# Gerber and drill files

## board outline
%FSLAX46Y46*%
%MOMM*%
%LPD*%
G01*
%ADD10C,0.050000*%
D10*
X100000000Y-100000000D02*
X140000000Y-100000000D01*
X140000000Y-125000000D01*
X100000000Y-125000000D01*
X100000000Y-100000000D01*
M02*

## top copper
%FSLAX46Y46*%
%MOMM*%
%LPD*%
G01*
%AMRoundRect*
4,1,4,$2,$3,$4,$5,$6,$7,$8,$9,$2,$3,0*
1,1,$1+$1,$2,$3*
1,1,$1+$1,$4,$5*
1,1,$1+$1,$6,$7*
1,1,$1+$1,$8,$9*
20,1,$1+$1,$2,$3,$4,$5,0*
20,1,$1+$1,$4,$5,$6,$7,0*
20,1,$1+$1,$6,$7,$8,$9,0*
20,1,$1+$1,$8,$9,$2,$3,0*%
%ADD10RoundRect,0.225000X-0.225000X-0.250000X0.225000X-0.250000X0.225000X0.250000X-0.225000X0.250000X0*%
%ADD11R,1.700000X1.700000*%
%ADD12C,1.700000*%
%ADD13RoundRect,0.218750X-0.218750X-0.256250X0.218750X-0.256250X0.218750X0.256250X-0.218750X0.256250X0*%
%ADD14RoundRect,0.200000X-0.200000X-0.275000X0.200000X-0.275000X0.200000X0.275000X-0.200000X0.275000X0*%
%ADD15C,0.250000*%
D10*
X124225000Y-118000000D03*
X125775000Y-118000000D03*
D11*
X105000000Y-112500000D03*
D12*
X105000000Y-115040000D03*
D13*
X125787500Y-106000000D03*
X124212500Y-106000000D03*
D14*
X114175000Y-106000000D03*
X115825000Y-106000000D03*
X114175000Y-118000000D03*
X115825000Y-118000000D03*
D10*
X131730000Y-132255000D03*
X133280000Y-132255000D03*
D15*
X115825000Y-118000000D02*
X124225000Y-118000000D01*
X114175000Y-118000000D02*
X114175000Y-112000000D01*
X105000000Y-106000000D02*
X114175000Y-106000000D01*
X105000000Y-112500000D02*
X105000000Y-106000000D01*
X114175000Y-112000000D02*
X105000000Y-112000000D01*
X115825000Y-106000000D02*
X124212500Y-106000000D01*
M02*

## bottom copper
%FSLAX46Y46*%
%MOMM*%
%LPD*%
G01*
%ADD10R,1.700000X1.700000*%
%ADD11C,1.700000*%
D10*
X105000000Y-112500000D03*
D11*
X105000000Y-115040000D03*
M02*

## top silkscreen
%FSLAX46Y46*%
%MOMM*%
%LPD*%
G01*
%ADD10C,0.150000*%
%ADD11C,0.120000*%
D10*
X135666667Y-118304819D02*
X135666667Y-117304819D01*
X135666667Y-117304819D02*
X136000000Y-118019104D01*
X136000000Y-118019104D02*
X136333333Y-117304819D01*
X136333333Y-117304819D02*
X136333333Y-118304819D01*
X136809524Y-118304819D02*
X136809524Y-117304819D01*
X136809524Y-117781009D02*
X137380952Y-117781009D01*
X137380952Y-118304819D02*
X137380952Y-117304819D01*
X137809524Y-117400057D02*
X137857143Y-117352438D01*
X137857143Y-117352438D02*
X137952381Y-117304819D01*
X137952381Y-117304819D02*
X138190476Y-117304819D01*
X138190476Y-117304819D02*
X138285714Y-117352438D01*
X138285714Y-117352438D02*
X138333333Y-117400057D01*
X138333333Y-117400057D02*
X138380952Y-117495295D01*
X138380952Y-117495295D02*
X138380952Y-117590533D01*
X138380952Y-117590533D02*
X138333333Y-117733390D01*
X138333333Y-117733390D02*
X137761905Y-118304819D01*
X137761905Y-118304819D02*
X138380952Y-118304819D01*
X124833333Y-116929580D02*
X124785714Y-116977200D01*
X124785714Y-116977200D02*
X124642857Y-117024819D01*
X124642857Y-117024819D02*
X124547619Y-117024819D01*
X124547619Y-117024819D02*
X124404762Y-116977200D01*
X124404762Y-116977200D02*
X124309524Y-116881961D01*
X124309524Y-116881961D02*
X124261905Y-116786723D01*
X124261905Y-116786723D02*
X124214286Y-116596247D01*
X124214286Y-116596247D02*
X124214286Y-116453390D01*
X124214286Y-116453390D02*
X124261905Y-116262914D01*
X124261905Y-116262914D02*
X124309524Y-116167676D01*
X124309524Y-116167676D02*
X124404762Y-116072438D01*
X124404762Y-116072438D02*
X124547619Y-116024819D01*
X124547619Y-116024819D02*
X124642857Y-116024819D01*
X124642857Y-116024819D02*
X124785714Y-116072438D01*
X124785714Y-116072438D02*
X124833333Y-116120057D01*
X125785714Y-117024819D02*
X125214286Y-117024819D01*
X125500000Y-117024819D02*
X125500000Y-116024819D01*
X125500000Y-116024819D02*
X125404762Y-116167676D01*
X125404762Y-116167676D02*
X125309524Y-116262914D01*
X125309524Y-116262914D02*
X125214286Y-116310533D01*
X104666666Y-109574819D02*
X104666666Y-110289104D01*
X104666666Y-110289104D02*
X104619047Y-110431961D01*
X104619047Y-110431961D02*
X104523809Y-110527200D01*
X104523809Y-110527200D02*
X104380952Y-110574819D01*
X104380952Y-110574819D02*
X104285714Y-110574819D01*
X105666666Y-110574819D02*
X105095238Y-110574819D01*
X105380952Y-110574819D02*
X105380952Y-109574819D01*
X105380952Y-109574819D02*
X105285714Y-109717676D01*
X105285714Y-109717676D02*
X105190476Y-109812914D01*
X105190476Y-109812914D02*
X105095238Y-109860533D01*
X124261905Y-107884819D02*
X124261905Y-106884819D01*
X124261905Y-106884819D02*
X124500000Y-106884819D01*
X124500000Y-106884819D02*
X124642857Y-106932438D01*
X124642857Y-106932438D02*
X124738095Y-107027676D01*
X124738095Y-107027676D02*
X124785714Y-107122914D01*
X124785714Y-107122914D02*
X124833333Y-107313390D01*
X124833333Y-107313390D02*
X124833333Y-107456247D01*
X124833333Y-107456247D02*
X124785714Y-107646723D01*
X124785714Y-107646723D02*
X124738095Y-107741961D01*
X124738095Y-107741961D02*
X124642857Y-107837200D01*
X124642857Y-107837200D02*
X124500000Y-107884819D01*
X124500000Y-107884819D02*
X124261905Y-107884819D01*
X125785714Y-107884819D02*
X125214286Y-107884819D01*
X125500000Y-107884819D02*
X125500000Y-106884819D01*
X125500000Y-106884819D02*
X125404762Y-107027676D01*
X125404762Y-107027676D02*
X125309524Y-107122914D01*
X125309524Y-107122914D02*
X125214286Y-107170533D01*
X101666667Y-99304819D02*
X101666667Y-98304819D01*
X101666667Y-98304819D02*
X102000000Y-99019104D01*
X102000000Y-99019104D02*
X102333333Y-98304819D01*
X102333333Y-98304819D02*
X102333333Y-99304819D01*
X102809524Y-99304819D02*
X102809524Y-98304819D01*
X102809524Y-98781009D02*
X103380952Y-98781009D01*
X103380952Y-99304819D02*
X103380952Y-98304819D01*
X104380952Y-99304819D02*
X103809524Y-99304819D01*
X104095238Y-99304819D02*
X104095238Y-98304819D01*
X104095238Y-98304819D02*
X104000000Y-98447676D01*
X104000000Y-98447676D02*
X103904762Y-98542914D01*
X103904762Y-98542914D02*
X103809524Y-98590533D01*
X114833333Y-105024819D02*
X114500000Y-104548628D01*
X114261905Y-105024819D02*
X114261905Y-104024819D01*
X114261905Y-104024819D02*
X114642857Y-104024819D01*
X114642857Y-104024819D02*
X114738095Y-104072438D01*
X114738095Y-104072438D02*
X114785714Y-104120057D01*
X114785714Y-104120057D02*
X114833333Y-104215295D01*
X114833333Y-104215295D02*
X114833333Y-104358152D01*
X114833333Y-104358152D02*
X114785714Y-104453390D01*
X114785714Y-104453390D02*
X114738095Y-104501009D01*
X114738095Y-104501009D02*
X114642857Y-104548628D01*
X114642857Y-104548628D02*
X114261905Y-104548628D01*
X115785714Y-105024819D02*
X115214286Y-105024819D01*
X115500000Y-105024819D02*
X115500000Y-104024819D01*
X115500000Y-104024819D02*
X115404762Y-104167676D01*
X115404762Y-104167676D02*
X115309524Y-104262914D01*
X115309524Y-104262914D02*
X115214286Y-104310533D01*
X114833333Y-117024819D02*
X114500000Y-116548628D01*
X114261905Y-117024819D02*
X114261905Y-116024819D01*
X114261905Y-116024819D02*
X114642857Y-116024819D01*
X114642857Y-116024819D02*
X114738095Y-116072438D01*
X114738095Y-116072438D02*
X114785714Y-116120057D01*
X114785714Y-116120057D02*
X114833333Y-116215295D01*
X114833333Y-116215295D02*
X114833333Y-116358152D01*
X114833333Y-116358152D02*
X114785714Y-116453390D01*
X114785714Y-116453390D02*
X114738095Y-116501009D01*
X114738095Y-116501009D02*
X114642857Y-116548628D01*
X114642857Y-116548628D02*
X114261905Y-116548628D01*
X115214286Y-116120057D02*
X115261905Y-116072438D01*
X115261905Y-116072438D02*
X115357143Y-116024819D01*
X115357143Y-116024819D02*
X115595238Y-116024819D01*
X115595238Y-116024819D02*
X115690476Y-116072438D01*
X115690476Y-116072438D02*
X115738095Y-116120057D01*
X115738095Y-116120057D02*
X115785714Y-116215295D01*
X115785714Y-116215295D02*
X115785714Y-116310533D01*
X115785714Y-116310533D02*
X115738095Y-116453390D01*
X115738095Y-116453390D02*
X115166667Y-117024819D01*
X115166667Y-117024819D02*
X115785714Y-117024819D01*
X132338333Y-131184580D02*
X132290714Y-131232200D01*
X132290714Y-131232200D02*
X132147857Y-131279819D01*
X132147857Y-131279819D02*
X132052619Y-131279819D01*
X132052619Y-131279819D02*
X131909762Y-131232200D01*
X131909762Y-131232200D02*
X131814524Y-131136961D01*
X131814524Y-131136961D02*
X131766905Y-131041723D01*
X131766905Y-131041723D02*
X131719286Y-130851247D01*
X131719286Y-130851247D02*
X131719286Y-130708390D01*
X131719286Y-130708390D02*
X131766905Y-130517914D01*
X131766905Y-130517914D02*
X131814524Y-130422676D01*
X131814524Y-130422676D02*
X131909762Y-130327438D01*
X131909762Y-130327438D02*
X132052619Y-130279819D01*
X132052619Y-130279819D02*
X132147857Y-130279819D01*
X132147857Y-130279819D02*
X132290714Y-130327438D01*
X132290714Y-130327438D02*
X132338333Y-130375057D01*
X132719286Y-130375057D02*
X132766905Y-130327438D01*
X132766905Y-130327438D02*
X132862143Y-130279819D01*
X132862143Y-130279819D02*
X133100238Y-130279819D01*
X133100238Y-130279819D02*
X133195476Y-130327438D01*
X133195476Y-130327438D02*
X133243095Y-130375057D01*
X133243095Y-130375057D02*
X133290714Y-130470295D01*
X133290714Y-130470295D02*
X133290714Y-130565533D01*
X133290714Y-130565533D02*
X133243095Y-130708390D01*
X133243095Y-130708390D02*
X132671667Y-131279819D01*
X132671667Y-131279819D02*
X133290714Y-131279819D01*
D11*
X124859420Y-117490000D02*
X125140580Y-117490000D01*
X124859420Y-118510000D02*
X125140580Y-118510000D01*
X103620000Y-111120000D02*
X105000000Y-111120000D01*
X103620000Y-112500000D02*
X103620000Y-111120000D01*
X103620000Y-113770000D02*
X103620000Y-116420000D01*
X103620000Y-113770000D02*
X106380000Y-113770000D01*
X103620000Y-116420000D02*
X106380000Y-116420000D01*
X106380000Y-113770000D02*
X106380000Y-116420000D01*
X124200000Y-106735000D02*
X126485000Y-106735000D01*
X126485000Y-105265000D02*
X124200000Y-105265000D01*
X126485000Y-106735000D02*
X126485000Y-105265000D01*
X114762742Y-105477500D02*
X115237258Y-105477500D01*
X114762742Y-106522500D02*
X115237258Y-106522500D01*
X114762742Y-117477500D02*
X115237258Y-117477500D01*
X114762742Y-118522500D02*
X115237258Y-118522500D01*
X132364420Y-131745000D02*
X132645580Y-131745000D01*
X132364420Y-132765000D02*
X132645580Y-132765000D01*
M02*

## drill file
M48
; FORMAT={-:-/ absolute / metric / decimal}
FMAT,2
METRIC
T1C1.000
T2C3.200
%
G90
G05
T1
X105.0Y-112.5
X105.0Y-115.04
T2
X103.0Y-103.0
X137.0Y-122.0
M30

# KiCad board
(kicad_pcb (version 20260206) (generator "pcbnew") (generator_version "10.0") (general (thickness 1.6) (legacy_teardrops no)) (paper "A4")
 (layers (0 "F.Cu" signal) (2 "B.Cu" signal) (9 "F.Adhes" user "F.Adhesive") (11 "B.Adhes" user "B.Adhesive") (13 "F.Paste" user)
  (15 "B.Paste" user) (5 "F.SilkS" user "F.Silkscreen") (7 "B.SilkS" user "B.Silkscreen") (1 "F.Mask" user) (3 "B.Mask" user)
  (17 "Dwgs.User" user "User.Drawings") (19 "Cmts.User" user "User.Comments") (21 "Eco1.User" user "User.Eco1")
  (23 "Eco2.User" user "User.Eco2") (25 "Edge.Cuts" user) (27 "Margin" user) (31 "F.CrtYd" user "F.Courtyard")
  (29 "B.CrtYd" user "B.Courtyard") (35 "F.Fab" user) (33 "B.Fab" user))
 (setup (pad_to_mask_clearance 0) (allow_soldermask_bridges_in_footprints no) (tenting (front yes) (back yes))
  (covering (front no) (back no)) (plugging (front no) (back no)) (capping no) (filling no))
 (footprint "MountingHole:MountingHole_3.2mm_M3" (layer "F.Cu") (at 137 122)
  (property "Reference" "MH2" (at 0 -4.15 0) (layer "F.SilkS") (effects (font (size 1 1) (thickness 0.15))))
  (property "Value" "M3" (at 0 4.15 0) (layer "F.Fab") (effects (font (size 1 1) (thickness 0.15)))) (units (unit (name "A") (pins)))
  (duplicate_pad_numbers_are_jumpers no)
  (pad "" np_thru_hole circle (at 0 0) (size 3.2 3.2) (drill 3.2) (layers "*.Cu" "*.Mask")))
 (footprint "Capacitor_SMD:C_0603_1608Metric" (layer "F.Cu") (at 125 118)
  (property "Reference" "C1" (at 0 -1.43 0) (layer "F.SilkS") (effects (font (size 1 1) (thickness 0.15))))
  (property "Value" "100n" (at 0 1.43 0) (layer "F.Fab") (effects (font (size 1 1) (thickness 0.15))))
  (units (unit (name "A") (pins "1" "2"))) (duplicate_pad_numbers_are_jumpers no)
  (fp_line (start -0.14058 -0.51) (end 0.14058 -0.51) (stroke (width 0.12) (type solid)) (layer "F.SilkS"))
  (fp_line (start -0.14058 0.51) (end 0.14058 0.51) (stroke (width 0.12) (type solid)) (layer "F.SilkS"))
  (pad "1" smd roundrect (at -0.775 0) (size 0.9 0.95) (layers "F.Cu" "F.Mask" "F.Paste") (roundrect_rratio 0.25) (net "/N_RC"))
  (pad "2" smd roundrect (at 0.775 0) (size 0.9 0.95) (layers "F.Cu" "F.Mask" "F.Paste") (roundrect_rratio 0.25) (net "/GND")))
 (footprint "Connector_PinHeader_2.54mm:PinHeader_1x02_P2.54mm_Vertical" (layer "F.Cu") (at 105 112.5)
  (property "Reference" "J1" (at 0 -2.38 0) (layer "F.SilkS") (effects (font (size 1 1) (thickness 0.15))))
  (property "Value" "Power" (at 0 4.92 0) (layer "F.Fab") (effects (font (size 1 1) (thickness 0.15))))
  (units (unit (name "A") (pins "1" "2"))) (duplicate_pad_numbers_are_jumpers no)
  (fp_line (start -1.38 -1.38) (end 0 -1.38) (stroke (width 0.12) (type solid)) (layer "F.SilkS"))
  (fp_line (start -1.38 0) (end -1.38 -1.38) (stroke (width 0.12) (type solid)) (layer "F.SilkS"))
  (fp_line (start -1.38 1.27) (end -1.38 3.92) (stroke (width 0.12) (type solid)) (layer "F.SilkS"))
  (fp_line (start -1.38 1.27) (end 1.38 1.27) (stroke (width 0.12) (type solid)) (layer "F.SilkS"))
  (fp_line (start -1.38 3.92) (end 1.38 3.92) (stroke (width 0.12) (type solid)) (layer "F.SilkS"))
  (fp_line (start 1.38 1.27) (end 1.38 3.92) (stroke (width 0.12) (type solid)) (layer "F.SilkS"))
  (pad "1" thru_hole rect (at 0 0) (size 1.7 1.7) (drill 1) (layers "*.Cu" "*.Mask") (remove_unused_layers no) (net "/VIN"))
  (pad "2" thru_hole circle (at 0 2.54) (size 1.7 1.7) (drill 1) (layers "*.Cu" "*.Mask") (remove_unused_layers no) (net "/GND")))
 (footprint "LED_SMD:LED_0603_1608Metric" (layer "F.Cu") (at 125 106 180)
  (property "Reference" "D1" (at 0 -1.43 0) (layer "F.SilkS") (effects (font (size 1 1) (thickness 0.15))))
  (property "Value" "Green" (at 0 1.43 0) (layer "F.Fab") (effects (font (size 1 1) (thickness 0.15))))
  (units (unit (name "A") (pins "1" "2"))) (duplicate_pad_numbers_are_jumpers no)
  (fp_line (start 0.8 -0.735) (end -1.485 -0.735) (stroke (width 0.12) (type solid)) (layer "F.SilkS"))
  (fp_line (start -1.485 0.735) (end 0.8 0.735) (stroke (width 0.12) (type solid)) (layer "F.SilkS"))
  (fp_line (start -1.485 -0.735) (end -1.485 0.735) (stroke (width 0.12) (type solid)) (layer "F.SilkS"))
  (pad "1" smd roundrect (at -0.7875 0) (size 0.875 0.95) (layers "F.Cu" "F.Mask" "F.Paste") (roundrect_rratio 0.25) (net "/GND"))
  (pad "2" smd roundrect (at 0.7875 0) (size 0.875 0.95) (layers "F.Cu" "F.Mask" "F.Paste") (roundrect_rratio 0.25) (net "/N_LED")))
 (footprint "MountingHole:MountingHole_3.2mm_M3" (layer "F.Cu") (at 103 103)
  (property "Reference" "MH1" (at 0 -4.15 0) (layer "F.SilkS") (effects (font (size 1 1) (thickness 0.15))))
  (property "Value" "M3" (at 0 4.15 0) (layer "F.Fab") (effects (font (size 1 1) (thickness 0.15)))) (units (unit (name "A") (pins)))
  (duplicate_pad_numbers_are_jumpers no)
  (pad "" np_thru_hole circle (at 0 0) (size 3.2 3.2) (drill 3.2) (layers "*.Cu" "*.Mask")))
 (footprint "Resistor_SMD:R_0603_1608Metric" (layer "F.Cu") (at 115 106)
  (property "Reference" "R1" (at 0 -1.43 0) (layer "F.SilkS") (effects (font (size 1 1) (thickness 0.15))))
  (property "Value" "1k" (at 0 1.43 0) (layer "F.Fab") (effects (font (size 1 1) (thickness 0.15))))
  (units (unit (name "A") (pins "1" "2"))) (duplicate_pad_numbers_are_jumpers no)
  (fp_line (start -0.237258 -0.5225) (end 0.237258 -0.5225) (stroke (width 0.12) (type solid)) (layer "F.SilkS"))
  (fp_line (start -0.237258 0.5225) (end 0.237258 0.5225) (stroke (width 0.12) (type solid)) (layer "F.SilkS"))
  (pad "1" smd roundrect (at -0.825 0) (size 0.8 0.95) (layers "F.Cu" "F.Mask" "F.Paste") (roundrect_rratio 0.25) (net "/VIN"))
  (pad "2" smd roundrect (at 0.825 0) (size 0.8 0.95) (layers "F.Cu" "F.Mask" "F.Paste") (roundrect_rratio 0.25) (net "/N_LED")))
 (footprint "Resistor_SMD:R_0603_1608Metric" (layer "F.Cu") (at 115 118)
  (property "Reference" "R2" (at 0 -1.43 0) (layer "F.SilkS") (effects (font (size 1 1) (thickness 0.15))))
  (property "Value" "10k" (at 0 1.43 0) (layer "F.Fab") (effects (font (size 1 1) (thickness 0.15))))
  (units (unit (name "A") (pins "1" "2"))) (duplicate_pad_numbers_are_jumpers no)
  (fp_line (start -0.237258 -0.5225) (end 0.237258 -0.5225) (stroke (width 0.12) (type solid)) (layer "F.SilkS"))
  (fp_line (start -0.237258 0.5225) (end 0.237258 0.5225) (stroke (width 0.12) (type solid)) (layer "F.SilkS"))
  (pad "1" smd roundrect (at -0.825 0) (size 0.8 0.95) (layers "F.Cu" "F.Mask" "F.Paste") (roundrect_rratio 0.25) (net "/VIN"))
  (pad "2" smd roundrect (at 0.825 0) (size 0.8 0.95) (layers "F.Cu" "F.Mask" "F.Paste") (roundrect_rratio 0.25) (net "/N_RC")))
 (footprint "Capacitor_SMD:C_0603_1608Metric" (layer "F.Cu") (at 132.505 132.255)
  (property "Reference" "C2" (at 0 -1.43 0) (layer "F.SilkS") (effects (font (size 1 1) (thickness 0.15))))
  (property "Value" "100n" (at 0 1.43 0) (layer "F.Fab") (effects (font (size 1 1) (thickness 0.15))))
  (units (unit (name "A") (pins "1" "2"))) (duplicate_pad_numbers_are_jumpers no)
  (fp_line (start -0.14058 -0.51) (end 0.14058 -0.51) (stroke (width 0.12) (type solid)) (layer "F.SilkS"))
  (fp_line (start -0.14058 0.51) (end 0.14058 0.51) (stroke (width 0.12) (type solid)) (layer "F.SilkS"))
  (pad "1" smd roundrect (at -0.775 0) (size 0.9 0.95) (layers "F.Cu" "F.Mask" "F.Paste") (roundrect_rratio 0.25) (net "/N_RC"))
  (pad "2" smd roundrect (at 0.775 0) (size 0.9 0.95) (layers "F.Cu" "F.Mask" "F.Paste") (roundrect_rratio 0.25) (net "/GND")))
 (gr_rect (start 100 100) (end 140 125) (stroke (width 0.05) (type default)) (fill no) (layer "Edge.Cuts"))
 (segment (start 115.825 118) (end 124.225 118) (width 0.25) (layer "F.Cu") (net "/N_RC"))
 (segment (start 114.175 118) (end 114.175 112) (width 0.25) (layer "F.Cu") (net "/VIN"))
 (segment (start 105 106) (end 114.175 106) (width 0.25) (layer "F.Cu") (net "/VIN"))
 (segment (start 105 112.5) (end 105 106) (width 0.25) (layer "F.Cu") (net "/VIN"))
 (segment (start 114.175 112) (end 105 112) (width 0.25) (layer "F.Cu") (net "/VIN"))
 (segment (start 115.825 106) (end 124.2125 106) (width 0.25) (layer "F.Cu") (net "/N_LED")))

